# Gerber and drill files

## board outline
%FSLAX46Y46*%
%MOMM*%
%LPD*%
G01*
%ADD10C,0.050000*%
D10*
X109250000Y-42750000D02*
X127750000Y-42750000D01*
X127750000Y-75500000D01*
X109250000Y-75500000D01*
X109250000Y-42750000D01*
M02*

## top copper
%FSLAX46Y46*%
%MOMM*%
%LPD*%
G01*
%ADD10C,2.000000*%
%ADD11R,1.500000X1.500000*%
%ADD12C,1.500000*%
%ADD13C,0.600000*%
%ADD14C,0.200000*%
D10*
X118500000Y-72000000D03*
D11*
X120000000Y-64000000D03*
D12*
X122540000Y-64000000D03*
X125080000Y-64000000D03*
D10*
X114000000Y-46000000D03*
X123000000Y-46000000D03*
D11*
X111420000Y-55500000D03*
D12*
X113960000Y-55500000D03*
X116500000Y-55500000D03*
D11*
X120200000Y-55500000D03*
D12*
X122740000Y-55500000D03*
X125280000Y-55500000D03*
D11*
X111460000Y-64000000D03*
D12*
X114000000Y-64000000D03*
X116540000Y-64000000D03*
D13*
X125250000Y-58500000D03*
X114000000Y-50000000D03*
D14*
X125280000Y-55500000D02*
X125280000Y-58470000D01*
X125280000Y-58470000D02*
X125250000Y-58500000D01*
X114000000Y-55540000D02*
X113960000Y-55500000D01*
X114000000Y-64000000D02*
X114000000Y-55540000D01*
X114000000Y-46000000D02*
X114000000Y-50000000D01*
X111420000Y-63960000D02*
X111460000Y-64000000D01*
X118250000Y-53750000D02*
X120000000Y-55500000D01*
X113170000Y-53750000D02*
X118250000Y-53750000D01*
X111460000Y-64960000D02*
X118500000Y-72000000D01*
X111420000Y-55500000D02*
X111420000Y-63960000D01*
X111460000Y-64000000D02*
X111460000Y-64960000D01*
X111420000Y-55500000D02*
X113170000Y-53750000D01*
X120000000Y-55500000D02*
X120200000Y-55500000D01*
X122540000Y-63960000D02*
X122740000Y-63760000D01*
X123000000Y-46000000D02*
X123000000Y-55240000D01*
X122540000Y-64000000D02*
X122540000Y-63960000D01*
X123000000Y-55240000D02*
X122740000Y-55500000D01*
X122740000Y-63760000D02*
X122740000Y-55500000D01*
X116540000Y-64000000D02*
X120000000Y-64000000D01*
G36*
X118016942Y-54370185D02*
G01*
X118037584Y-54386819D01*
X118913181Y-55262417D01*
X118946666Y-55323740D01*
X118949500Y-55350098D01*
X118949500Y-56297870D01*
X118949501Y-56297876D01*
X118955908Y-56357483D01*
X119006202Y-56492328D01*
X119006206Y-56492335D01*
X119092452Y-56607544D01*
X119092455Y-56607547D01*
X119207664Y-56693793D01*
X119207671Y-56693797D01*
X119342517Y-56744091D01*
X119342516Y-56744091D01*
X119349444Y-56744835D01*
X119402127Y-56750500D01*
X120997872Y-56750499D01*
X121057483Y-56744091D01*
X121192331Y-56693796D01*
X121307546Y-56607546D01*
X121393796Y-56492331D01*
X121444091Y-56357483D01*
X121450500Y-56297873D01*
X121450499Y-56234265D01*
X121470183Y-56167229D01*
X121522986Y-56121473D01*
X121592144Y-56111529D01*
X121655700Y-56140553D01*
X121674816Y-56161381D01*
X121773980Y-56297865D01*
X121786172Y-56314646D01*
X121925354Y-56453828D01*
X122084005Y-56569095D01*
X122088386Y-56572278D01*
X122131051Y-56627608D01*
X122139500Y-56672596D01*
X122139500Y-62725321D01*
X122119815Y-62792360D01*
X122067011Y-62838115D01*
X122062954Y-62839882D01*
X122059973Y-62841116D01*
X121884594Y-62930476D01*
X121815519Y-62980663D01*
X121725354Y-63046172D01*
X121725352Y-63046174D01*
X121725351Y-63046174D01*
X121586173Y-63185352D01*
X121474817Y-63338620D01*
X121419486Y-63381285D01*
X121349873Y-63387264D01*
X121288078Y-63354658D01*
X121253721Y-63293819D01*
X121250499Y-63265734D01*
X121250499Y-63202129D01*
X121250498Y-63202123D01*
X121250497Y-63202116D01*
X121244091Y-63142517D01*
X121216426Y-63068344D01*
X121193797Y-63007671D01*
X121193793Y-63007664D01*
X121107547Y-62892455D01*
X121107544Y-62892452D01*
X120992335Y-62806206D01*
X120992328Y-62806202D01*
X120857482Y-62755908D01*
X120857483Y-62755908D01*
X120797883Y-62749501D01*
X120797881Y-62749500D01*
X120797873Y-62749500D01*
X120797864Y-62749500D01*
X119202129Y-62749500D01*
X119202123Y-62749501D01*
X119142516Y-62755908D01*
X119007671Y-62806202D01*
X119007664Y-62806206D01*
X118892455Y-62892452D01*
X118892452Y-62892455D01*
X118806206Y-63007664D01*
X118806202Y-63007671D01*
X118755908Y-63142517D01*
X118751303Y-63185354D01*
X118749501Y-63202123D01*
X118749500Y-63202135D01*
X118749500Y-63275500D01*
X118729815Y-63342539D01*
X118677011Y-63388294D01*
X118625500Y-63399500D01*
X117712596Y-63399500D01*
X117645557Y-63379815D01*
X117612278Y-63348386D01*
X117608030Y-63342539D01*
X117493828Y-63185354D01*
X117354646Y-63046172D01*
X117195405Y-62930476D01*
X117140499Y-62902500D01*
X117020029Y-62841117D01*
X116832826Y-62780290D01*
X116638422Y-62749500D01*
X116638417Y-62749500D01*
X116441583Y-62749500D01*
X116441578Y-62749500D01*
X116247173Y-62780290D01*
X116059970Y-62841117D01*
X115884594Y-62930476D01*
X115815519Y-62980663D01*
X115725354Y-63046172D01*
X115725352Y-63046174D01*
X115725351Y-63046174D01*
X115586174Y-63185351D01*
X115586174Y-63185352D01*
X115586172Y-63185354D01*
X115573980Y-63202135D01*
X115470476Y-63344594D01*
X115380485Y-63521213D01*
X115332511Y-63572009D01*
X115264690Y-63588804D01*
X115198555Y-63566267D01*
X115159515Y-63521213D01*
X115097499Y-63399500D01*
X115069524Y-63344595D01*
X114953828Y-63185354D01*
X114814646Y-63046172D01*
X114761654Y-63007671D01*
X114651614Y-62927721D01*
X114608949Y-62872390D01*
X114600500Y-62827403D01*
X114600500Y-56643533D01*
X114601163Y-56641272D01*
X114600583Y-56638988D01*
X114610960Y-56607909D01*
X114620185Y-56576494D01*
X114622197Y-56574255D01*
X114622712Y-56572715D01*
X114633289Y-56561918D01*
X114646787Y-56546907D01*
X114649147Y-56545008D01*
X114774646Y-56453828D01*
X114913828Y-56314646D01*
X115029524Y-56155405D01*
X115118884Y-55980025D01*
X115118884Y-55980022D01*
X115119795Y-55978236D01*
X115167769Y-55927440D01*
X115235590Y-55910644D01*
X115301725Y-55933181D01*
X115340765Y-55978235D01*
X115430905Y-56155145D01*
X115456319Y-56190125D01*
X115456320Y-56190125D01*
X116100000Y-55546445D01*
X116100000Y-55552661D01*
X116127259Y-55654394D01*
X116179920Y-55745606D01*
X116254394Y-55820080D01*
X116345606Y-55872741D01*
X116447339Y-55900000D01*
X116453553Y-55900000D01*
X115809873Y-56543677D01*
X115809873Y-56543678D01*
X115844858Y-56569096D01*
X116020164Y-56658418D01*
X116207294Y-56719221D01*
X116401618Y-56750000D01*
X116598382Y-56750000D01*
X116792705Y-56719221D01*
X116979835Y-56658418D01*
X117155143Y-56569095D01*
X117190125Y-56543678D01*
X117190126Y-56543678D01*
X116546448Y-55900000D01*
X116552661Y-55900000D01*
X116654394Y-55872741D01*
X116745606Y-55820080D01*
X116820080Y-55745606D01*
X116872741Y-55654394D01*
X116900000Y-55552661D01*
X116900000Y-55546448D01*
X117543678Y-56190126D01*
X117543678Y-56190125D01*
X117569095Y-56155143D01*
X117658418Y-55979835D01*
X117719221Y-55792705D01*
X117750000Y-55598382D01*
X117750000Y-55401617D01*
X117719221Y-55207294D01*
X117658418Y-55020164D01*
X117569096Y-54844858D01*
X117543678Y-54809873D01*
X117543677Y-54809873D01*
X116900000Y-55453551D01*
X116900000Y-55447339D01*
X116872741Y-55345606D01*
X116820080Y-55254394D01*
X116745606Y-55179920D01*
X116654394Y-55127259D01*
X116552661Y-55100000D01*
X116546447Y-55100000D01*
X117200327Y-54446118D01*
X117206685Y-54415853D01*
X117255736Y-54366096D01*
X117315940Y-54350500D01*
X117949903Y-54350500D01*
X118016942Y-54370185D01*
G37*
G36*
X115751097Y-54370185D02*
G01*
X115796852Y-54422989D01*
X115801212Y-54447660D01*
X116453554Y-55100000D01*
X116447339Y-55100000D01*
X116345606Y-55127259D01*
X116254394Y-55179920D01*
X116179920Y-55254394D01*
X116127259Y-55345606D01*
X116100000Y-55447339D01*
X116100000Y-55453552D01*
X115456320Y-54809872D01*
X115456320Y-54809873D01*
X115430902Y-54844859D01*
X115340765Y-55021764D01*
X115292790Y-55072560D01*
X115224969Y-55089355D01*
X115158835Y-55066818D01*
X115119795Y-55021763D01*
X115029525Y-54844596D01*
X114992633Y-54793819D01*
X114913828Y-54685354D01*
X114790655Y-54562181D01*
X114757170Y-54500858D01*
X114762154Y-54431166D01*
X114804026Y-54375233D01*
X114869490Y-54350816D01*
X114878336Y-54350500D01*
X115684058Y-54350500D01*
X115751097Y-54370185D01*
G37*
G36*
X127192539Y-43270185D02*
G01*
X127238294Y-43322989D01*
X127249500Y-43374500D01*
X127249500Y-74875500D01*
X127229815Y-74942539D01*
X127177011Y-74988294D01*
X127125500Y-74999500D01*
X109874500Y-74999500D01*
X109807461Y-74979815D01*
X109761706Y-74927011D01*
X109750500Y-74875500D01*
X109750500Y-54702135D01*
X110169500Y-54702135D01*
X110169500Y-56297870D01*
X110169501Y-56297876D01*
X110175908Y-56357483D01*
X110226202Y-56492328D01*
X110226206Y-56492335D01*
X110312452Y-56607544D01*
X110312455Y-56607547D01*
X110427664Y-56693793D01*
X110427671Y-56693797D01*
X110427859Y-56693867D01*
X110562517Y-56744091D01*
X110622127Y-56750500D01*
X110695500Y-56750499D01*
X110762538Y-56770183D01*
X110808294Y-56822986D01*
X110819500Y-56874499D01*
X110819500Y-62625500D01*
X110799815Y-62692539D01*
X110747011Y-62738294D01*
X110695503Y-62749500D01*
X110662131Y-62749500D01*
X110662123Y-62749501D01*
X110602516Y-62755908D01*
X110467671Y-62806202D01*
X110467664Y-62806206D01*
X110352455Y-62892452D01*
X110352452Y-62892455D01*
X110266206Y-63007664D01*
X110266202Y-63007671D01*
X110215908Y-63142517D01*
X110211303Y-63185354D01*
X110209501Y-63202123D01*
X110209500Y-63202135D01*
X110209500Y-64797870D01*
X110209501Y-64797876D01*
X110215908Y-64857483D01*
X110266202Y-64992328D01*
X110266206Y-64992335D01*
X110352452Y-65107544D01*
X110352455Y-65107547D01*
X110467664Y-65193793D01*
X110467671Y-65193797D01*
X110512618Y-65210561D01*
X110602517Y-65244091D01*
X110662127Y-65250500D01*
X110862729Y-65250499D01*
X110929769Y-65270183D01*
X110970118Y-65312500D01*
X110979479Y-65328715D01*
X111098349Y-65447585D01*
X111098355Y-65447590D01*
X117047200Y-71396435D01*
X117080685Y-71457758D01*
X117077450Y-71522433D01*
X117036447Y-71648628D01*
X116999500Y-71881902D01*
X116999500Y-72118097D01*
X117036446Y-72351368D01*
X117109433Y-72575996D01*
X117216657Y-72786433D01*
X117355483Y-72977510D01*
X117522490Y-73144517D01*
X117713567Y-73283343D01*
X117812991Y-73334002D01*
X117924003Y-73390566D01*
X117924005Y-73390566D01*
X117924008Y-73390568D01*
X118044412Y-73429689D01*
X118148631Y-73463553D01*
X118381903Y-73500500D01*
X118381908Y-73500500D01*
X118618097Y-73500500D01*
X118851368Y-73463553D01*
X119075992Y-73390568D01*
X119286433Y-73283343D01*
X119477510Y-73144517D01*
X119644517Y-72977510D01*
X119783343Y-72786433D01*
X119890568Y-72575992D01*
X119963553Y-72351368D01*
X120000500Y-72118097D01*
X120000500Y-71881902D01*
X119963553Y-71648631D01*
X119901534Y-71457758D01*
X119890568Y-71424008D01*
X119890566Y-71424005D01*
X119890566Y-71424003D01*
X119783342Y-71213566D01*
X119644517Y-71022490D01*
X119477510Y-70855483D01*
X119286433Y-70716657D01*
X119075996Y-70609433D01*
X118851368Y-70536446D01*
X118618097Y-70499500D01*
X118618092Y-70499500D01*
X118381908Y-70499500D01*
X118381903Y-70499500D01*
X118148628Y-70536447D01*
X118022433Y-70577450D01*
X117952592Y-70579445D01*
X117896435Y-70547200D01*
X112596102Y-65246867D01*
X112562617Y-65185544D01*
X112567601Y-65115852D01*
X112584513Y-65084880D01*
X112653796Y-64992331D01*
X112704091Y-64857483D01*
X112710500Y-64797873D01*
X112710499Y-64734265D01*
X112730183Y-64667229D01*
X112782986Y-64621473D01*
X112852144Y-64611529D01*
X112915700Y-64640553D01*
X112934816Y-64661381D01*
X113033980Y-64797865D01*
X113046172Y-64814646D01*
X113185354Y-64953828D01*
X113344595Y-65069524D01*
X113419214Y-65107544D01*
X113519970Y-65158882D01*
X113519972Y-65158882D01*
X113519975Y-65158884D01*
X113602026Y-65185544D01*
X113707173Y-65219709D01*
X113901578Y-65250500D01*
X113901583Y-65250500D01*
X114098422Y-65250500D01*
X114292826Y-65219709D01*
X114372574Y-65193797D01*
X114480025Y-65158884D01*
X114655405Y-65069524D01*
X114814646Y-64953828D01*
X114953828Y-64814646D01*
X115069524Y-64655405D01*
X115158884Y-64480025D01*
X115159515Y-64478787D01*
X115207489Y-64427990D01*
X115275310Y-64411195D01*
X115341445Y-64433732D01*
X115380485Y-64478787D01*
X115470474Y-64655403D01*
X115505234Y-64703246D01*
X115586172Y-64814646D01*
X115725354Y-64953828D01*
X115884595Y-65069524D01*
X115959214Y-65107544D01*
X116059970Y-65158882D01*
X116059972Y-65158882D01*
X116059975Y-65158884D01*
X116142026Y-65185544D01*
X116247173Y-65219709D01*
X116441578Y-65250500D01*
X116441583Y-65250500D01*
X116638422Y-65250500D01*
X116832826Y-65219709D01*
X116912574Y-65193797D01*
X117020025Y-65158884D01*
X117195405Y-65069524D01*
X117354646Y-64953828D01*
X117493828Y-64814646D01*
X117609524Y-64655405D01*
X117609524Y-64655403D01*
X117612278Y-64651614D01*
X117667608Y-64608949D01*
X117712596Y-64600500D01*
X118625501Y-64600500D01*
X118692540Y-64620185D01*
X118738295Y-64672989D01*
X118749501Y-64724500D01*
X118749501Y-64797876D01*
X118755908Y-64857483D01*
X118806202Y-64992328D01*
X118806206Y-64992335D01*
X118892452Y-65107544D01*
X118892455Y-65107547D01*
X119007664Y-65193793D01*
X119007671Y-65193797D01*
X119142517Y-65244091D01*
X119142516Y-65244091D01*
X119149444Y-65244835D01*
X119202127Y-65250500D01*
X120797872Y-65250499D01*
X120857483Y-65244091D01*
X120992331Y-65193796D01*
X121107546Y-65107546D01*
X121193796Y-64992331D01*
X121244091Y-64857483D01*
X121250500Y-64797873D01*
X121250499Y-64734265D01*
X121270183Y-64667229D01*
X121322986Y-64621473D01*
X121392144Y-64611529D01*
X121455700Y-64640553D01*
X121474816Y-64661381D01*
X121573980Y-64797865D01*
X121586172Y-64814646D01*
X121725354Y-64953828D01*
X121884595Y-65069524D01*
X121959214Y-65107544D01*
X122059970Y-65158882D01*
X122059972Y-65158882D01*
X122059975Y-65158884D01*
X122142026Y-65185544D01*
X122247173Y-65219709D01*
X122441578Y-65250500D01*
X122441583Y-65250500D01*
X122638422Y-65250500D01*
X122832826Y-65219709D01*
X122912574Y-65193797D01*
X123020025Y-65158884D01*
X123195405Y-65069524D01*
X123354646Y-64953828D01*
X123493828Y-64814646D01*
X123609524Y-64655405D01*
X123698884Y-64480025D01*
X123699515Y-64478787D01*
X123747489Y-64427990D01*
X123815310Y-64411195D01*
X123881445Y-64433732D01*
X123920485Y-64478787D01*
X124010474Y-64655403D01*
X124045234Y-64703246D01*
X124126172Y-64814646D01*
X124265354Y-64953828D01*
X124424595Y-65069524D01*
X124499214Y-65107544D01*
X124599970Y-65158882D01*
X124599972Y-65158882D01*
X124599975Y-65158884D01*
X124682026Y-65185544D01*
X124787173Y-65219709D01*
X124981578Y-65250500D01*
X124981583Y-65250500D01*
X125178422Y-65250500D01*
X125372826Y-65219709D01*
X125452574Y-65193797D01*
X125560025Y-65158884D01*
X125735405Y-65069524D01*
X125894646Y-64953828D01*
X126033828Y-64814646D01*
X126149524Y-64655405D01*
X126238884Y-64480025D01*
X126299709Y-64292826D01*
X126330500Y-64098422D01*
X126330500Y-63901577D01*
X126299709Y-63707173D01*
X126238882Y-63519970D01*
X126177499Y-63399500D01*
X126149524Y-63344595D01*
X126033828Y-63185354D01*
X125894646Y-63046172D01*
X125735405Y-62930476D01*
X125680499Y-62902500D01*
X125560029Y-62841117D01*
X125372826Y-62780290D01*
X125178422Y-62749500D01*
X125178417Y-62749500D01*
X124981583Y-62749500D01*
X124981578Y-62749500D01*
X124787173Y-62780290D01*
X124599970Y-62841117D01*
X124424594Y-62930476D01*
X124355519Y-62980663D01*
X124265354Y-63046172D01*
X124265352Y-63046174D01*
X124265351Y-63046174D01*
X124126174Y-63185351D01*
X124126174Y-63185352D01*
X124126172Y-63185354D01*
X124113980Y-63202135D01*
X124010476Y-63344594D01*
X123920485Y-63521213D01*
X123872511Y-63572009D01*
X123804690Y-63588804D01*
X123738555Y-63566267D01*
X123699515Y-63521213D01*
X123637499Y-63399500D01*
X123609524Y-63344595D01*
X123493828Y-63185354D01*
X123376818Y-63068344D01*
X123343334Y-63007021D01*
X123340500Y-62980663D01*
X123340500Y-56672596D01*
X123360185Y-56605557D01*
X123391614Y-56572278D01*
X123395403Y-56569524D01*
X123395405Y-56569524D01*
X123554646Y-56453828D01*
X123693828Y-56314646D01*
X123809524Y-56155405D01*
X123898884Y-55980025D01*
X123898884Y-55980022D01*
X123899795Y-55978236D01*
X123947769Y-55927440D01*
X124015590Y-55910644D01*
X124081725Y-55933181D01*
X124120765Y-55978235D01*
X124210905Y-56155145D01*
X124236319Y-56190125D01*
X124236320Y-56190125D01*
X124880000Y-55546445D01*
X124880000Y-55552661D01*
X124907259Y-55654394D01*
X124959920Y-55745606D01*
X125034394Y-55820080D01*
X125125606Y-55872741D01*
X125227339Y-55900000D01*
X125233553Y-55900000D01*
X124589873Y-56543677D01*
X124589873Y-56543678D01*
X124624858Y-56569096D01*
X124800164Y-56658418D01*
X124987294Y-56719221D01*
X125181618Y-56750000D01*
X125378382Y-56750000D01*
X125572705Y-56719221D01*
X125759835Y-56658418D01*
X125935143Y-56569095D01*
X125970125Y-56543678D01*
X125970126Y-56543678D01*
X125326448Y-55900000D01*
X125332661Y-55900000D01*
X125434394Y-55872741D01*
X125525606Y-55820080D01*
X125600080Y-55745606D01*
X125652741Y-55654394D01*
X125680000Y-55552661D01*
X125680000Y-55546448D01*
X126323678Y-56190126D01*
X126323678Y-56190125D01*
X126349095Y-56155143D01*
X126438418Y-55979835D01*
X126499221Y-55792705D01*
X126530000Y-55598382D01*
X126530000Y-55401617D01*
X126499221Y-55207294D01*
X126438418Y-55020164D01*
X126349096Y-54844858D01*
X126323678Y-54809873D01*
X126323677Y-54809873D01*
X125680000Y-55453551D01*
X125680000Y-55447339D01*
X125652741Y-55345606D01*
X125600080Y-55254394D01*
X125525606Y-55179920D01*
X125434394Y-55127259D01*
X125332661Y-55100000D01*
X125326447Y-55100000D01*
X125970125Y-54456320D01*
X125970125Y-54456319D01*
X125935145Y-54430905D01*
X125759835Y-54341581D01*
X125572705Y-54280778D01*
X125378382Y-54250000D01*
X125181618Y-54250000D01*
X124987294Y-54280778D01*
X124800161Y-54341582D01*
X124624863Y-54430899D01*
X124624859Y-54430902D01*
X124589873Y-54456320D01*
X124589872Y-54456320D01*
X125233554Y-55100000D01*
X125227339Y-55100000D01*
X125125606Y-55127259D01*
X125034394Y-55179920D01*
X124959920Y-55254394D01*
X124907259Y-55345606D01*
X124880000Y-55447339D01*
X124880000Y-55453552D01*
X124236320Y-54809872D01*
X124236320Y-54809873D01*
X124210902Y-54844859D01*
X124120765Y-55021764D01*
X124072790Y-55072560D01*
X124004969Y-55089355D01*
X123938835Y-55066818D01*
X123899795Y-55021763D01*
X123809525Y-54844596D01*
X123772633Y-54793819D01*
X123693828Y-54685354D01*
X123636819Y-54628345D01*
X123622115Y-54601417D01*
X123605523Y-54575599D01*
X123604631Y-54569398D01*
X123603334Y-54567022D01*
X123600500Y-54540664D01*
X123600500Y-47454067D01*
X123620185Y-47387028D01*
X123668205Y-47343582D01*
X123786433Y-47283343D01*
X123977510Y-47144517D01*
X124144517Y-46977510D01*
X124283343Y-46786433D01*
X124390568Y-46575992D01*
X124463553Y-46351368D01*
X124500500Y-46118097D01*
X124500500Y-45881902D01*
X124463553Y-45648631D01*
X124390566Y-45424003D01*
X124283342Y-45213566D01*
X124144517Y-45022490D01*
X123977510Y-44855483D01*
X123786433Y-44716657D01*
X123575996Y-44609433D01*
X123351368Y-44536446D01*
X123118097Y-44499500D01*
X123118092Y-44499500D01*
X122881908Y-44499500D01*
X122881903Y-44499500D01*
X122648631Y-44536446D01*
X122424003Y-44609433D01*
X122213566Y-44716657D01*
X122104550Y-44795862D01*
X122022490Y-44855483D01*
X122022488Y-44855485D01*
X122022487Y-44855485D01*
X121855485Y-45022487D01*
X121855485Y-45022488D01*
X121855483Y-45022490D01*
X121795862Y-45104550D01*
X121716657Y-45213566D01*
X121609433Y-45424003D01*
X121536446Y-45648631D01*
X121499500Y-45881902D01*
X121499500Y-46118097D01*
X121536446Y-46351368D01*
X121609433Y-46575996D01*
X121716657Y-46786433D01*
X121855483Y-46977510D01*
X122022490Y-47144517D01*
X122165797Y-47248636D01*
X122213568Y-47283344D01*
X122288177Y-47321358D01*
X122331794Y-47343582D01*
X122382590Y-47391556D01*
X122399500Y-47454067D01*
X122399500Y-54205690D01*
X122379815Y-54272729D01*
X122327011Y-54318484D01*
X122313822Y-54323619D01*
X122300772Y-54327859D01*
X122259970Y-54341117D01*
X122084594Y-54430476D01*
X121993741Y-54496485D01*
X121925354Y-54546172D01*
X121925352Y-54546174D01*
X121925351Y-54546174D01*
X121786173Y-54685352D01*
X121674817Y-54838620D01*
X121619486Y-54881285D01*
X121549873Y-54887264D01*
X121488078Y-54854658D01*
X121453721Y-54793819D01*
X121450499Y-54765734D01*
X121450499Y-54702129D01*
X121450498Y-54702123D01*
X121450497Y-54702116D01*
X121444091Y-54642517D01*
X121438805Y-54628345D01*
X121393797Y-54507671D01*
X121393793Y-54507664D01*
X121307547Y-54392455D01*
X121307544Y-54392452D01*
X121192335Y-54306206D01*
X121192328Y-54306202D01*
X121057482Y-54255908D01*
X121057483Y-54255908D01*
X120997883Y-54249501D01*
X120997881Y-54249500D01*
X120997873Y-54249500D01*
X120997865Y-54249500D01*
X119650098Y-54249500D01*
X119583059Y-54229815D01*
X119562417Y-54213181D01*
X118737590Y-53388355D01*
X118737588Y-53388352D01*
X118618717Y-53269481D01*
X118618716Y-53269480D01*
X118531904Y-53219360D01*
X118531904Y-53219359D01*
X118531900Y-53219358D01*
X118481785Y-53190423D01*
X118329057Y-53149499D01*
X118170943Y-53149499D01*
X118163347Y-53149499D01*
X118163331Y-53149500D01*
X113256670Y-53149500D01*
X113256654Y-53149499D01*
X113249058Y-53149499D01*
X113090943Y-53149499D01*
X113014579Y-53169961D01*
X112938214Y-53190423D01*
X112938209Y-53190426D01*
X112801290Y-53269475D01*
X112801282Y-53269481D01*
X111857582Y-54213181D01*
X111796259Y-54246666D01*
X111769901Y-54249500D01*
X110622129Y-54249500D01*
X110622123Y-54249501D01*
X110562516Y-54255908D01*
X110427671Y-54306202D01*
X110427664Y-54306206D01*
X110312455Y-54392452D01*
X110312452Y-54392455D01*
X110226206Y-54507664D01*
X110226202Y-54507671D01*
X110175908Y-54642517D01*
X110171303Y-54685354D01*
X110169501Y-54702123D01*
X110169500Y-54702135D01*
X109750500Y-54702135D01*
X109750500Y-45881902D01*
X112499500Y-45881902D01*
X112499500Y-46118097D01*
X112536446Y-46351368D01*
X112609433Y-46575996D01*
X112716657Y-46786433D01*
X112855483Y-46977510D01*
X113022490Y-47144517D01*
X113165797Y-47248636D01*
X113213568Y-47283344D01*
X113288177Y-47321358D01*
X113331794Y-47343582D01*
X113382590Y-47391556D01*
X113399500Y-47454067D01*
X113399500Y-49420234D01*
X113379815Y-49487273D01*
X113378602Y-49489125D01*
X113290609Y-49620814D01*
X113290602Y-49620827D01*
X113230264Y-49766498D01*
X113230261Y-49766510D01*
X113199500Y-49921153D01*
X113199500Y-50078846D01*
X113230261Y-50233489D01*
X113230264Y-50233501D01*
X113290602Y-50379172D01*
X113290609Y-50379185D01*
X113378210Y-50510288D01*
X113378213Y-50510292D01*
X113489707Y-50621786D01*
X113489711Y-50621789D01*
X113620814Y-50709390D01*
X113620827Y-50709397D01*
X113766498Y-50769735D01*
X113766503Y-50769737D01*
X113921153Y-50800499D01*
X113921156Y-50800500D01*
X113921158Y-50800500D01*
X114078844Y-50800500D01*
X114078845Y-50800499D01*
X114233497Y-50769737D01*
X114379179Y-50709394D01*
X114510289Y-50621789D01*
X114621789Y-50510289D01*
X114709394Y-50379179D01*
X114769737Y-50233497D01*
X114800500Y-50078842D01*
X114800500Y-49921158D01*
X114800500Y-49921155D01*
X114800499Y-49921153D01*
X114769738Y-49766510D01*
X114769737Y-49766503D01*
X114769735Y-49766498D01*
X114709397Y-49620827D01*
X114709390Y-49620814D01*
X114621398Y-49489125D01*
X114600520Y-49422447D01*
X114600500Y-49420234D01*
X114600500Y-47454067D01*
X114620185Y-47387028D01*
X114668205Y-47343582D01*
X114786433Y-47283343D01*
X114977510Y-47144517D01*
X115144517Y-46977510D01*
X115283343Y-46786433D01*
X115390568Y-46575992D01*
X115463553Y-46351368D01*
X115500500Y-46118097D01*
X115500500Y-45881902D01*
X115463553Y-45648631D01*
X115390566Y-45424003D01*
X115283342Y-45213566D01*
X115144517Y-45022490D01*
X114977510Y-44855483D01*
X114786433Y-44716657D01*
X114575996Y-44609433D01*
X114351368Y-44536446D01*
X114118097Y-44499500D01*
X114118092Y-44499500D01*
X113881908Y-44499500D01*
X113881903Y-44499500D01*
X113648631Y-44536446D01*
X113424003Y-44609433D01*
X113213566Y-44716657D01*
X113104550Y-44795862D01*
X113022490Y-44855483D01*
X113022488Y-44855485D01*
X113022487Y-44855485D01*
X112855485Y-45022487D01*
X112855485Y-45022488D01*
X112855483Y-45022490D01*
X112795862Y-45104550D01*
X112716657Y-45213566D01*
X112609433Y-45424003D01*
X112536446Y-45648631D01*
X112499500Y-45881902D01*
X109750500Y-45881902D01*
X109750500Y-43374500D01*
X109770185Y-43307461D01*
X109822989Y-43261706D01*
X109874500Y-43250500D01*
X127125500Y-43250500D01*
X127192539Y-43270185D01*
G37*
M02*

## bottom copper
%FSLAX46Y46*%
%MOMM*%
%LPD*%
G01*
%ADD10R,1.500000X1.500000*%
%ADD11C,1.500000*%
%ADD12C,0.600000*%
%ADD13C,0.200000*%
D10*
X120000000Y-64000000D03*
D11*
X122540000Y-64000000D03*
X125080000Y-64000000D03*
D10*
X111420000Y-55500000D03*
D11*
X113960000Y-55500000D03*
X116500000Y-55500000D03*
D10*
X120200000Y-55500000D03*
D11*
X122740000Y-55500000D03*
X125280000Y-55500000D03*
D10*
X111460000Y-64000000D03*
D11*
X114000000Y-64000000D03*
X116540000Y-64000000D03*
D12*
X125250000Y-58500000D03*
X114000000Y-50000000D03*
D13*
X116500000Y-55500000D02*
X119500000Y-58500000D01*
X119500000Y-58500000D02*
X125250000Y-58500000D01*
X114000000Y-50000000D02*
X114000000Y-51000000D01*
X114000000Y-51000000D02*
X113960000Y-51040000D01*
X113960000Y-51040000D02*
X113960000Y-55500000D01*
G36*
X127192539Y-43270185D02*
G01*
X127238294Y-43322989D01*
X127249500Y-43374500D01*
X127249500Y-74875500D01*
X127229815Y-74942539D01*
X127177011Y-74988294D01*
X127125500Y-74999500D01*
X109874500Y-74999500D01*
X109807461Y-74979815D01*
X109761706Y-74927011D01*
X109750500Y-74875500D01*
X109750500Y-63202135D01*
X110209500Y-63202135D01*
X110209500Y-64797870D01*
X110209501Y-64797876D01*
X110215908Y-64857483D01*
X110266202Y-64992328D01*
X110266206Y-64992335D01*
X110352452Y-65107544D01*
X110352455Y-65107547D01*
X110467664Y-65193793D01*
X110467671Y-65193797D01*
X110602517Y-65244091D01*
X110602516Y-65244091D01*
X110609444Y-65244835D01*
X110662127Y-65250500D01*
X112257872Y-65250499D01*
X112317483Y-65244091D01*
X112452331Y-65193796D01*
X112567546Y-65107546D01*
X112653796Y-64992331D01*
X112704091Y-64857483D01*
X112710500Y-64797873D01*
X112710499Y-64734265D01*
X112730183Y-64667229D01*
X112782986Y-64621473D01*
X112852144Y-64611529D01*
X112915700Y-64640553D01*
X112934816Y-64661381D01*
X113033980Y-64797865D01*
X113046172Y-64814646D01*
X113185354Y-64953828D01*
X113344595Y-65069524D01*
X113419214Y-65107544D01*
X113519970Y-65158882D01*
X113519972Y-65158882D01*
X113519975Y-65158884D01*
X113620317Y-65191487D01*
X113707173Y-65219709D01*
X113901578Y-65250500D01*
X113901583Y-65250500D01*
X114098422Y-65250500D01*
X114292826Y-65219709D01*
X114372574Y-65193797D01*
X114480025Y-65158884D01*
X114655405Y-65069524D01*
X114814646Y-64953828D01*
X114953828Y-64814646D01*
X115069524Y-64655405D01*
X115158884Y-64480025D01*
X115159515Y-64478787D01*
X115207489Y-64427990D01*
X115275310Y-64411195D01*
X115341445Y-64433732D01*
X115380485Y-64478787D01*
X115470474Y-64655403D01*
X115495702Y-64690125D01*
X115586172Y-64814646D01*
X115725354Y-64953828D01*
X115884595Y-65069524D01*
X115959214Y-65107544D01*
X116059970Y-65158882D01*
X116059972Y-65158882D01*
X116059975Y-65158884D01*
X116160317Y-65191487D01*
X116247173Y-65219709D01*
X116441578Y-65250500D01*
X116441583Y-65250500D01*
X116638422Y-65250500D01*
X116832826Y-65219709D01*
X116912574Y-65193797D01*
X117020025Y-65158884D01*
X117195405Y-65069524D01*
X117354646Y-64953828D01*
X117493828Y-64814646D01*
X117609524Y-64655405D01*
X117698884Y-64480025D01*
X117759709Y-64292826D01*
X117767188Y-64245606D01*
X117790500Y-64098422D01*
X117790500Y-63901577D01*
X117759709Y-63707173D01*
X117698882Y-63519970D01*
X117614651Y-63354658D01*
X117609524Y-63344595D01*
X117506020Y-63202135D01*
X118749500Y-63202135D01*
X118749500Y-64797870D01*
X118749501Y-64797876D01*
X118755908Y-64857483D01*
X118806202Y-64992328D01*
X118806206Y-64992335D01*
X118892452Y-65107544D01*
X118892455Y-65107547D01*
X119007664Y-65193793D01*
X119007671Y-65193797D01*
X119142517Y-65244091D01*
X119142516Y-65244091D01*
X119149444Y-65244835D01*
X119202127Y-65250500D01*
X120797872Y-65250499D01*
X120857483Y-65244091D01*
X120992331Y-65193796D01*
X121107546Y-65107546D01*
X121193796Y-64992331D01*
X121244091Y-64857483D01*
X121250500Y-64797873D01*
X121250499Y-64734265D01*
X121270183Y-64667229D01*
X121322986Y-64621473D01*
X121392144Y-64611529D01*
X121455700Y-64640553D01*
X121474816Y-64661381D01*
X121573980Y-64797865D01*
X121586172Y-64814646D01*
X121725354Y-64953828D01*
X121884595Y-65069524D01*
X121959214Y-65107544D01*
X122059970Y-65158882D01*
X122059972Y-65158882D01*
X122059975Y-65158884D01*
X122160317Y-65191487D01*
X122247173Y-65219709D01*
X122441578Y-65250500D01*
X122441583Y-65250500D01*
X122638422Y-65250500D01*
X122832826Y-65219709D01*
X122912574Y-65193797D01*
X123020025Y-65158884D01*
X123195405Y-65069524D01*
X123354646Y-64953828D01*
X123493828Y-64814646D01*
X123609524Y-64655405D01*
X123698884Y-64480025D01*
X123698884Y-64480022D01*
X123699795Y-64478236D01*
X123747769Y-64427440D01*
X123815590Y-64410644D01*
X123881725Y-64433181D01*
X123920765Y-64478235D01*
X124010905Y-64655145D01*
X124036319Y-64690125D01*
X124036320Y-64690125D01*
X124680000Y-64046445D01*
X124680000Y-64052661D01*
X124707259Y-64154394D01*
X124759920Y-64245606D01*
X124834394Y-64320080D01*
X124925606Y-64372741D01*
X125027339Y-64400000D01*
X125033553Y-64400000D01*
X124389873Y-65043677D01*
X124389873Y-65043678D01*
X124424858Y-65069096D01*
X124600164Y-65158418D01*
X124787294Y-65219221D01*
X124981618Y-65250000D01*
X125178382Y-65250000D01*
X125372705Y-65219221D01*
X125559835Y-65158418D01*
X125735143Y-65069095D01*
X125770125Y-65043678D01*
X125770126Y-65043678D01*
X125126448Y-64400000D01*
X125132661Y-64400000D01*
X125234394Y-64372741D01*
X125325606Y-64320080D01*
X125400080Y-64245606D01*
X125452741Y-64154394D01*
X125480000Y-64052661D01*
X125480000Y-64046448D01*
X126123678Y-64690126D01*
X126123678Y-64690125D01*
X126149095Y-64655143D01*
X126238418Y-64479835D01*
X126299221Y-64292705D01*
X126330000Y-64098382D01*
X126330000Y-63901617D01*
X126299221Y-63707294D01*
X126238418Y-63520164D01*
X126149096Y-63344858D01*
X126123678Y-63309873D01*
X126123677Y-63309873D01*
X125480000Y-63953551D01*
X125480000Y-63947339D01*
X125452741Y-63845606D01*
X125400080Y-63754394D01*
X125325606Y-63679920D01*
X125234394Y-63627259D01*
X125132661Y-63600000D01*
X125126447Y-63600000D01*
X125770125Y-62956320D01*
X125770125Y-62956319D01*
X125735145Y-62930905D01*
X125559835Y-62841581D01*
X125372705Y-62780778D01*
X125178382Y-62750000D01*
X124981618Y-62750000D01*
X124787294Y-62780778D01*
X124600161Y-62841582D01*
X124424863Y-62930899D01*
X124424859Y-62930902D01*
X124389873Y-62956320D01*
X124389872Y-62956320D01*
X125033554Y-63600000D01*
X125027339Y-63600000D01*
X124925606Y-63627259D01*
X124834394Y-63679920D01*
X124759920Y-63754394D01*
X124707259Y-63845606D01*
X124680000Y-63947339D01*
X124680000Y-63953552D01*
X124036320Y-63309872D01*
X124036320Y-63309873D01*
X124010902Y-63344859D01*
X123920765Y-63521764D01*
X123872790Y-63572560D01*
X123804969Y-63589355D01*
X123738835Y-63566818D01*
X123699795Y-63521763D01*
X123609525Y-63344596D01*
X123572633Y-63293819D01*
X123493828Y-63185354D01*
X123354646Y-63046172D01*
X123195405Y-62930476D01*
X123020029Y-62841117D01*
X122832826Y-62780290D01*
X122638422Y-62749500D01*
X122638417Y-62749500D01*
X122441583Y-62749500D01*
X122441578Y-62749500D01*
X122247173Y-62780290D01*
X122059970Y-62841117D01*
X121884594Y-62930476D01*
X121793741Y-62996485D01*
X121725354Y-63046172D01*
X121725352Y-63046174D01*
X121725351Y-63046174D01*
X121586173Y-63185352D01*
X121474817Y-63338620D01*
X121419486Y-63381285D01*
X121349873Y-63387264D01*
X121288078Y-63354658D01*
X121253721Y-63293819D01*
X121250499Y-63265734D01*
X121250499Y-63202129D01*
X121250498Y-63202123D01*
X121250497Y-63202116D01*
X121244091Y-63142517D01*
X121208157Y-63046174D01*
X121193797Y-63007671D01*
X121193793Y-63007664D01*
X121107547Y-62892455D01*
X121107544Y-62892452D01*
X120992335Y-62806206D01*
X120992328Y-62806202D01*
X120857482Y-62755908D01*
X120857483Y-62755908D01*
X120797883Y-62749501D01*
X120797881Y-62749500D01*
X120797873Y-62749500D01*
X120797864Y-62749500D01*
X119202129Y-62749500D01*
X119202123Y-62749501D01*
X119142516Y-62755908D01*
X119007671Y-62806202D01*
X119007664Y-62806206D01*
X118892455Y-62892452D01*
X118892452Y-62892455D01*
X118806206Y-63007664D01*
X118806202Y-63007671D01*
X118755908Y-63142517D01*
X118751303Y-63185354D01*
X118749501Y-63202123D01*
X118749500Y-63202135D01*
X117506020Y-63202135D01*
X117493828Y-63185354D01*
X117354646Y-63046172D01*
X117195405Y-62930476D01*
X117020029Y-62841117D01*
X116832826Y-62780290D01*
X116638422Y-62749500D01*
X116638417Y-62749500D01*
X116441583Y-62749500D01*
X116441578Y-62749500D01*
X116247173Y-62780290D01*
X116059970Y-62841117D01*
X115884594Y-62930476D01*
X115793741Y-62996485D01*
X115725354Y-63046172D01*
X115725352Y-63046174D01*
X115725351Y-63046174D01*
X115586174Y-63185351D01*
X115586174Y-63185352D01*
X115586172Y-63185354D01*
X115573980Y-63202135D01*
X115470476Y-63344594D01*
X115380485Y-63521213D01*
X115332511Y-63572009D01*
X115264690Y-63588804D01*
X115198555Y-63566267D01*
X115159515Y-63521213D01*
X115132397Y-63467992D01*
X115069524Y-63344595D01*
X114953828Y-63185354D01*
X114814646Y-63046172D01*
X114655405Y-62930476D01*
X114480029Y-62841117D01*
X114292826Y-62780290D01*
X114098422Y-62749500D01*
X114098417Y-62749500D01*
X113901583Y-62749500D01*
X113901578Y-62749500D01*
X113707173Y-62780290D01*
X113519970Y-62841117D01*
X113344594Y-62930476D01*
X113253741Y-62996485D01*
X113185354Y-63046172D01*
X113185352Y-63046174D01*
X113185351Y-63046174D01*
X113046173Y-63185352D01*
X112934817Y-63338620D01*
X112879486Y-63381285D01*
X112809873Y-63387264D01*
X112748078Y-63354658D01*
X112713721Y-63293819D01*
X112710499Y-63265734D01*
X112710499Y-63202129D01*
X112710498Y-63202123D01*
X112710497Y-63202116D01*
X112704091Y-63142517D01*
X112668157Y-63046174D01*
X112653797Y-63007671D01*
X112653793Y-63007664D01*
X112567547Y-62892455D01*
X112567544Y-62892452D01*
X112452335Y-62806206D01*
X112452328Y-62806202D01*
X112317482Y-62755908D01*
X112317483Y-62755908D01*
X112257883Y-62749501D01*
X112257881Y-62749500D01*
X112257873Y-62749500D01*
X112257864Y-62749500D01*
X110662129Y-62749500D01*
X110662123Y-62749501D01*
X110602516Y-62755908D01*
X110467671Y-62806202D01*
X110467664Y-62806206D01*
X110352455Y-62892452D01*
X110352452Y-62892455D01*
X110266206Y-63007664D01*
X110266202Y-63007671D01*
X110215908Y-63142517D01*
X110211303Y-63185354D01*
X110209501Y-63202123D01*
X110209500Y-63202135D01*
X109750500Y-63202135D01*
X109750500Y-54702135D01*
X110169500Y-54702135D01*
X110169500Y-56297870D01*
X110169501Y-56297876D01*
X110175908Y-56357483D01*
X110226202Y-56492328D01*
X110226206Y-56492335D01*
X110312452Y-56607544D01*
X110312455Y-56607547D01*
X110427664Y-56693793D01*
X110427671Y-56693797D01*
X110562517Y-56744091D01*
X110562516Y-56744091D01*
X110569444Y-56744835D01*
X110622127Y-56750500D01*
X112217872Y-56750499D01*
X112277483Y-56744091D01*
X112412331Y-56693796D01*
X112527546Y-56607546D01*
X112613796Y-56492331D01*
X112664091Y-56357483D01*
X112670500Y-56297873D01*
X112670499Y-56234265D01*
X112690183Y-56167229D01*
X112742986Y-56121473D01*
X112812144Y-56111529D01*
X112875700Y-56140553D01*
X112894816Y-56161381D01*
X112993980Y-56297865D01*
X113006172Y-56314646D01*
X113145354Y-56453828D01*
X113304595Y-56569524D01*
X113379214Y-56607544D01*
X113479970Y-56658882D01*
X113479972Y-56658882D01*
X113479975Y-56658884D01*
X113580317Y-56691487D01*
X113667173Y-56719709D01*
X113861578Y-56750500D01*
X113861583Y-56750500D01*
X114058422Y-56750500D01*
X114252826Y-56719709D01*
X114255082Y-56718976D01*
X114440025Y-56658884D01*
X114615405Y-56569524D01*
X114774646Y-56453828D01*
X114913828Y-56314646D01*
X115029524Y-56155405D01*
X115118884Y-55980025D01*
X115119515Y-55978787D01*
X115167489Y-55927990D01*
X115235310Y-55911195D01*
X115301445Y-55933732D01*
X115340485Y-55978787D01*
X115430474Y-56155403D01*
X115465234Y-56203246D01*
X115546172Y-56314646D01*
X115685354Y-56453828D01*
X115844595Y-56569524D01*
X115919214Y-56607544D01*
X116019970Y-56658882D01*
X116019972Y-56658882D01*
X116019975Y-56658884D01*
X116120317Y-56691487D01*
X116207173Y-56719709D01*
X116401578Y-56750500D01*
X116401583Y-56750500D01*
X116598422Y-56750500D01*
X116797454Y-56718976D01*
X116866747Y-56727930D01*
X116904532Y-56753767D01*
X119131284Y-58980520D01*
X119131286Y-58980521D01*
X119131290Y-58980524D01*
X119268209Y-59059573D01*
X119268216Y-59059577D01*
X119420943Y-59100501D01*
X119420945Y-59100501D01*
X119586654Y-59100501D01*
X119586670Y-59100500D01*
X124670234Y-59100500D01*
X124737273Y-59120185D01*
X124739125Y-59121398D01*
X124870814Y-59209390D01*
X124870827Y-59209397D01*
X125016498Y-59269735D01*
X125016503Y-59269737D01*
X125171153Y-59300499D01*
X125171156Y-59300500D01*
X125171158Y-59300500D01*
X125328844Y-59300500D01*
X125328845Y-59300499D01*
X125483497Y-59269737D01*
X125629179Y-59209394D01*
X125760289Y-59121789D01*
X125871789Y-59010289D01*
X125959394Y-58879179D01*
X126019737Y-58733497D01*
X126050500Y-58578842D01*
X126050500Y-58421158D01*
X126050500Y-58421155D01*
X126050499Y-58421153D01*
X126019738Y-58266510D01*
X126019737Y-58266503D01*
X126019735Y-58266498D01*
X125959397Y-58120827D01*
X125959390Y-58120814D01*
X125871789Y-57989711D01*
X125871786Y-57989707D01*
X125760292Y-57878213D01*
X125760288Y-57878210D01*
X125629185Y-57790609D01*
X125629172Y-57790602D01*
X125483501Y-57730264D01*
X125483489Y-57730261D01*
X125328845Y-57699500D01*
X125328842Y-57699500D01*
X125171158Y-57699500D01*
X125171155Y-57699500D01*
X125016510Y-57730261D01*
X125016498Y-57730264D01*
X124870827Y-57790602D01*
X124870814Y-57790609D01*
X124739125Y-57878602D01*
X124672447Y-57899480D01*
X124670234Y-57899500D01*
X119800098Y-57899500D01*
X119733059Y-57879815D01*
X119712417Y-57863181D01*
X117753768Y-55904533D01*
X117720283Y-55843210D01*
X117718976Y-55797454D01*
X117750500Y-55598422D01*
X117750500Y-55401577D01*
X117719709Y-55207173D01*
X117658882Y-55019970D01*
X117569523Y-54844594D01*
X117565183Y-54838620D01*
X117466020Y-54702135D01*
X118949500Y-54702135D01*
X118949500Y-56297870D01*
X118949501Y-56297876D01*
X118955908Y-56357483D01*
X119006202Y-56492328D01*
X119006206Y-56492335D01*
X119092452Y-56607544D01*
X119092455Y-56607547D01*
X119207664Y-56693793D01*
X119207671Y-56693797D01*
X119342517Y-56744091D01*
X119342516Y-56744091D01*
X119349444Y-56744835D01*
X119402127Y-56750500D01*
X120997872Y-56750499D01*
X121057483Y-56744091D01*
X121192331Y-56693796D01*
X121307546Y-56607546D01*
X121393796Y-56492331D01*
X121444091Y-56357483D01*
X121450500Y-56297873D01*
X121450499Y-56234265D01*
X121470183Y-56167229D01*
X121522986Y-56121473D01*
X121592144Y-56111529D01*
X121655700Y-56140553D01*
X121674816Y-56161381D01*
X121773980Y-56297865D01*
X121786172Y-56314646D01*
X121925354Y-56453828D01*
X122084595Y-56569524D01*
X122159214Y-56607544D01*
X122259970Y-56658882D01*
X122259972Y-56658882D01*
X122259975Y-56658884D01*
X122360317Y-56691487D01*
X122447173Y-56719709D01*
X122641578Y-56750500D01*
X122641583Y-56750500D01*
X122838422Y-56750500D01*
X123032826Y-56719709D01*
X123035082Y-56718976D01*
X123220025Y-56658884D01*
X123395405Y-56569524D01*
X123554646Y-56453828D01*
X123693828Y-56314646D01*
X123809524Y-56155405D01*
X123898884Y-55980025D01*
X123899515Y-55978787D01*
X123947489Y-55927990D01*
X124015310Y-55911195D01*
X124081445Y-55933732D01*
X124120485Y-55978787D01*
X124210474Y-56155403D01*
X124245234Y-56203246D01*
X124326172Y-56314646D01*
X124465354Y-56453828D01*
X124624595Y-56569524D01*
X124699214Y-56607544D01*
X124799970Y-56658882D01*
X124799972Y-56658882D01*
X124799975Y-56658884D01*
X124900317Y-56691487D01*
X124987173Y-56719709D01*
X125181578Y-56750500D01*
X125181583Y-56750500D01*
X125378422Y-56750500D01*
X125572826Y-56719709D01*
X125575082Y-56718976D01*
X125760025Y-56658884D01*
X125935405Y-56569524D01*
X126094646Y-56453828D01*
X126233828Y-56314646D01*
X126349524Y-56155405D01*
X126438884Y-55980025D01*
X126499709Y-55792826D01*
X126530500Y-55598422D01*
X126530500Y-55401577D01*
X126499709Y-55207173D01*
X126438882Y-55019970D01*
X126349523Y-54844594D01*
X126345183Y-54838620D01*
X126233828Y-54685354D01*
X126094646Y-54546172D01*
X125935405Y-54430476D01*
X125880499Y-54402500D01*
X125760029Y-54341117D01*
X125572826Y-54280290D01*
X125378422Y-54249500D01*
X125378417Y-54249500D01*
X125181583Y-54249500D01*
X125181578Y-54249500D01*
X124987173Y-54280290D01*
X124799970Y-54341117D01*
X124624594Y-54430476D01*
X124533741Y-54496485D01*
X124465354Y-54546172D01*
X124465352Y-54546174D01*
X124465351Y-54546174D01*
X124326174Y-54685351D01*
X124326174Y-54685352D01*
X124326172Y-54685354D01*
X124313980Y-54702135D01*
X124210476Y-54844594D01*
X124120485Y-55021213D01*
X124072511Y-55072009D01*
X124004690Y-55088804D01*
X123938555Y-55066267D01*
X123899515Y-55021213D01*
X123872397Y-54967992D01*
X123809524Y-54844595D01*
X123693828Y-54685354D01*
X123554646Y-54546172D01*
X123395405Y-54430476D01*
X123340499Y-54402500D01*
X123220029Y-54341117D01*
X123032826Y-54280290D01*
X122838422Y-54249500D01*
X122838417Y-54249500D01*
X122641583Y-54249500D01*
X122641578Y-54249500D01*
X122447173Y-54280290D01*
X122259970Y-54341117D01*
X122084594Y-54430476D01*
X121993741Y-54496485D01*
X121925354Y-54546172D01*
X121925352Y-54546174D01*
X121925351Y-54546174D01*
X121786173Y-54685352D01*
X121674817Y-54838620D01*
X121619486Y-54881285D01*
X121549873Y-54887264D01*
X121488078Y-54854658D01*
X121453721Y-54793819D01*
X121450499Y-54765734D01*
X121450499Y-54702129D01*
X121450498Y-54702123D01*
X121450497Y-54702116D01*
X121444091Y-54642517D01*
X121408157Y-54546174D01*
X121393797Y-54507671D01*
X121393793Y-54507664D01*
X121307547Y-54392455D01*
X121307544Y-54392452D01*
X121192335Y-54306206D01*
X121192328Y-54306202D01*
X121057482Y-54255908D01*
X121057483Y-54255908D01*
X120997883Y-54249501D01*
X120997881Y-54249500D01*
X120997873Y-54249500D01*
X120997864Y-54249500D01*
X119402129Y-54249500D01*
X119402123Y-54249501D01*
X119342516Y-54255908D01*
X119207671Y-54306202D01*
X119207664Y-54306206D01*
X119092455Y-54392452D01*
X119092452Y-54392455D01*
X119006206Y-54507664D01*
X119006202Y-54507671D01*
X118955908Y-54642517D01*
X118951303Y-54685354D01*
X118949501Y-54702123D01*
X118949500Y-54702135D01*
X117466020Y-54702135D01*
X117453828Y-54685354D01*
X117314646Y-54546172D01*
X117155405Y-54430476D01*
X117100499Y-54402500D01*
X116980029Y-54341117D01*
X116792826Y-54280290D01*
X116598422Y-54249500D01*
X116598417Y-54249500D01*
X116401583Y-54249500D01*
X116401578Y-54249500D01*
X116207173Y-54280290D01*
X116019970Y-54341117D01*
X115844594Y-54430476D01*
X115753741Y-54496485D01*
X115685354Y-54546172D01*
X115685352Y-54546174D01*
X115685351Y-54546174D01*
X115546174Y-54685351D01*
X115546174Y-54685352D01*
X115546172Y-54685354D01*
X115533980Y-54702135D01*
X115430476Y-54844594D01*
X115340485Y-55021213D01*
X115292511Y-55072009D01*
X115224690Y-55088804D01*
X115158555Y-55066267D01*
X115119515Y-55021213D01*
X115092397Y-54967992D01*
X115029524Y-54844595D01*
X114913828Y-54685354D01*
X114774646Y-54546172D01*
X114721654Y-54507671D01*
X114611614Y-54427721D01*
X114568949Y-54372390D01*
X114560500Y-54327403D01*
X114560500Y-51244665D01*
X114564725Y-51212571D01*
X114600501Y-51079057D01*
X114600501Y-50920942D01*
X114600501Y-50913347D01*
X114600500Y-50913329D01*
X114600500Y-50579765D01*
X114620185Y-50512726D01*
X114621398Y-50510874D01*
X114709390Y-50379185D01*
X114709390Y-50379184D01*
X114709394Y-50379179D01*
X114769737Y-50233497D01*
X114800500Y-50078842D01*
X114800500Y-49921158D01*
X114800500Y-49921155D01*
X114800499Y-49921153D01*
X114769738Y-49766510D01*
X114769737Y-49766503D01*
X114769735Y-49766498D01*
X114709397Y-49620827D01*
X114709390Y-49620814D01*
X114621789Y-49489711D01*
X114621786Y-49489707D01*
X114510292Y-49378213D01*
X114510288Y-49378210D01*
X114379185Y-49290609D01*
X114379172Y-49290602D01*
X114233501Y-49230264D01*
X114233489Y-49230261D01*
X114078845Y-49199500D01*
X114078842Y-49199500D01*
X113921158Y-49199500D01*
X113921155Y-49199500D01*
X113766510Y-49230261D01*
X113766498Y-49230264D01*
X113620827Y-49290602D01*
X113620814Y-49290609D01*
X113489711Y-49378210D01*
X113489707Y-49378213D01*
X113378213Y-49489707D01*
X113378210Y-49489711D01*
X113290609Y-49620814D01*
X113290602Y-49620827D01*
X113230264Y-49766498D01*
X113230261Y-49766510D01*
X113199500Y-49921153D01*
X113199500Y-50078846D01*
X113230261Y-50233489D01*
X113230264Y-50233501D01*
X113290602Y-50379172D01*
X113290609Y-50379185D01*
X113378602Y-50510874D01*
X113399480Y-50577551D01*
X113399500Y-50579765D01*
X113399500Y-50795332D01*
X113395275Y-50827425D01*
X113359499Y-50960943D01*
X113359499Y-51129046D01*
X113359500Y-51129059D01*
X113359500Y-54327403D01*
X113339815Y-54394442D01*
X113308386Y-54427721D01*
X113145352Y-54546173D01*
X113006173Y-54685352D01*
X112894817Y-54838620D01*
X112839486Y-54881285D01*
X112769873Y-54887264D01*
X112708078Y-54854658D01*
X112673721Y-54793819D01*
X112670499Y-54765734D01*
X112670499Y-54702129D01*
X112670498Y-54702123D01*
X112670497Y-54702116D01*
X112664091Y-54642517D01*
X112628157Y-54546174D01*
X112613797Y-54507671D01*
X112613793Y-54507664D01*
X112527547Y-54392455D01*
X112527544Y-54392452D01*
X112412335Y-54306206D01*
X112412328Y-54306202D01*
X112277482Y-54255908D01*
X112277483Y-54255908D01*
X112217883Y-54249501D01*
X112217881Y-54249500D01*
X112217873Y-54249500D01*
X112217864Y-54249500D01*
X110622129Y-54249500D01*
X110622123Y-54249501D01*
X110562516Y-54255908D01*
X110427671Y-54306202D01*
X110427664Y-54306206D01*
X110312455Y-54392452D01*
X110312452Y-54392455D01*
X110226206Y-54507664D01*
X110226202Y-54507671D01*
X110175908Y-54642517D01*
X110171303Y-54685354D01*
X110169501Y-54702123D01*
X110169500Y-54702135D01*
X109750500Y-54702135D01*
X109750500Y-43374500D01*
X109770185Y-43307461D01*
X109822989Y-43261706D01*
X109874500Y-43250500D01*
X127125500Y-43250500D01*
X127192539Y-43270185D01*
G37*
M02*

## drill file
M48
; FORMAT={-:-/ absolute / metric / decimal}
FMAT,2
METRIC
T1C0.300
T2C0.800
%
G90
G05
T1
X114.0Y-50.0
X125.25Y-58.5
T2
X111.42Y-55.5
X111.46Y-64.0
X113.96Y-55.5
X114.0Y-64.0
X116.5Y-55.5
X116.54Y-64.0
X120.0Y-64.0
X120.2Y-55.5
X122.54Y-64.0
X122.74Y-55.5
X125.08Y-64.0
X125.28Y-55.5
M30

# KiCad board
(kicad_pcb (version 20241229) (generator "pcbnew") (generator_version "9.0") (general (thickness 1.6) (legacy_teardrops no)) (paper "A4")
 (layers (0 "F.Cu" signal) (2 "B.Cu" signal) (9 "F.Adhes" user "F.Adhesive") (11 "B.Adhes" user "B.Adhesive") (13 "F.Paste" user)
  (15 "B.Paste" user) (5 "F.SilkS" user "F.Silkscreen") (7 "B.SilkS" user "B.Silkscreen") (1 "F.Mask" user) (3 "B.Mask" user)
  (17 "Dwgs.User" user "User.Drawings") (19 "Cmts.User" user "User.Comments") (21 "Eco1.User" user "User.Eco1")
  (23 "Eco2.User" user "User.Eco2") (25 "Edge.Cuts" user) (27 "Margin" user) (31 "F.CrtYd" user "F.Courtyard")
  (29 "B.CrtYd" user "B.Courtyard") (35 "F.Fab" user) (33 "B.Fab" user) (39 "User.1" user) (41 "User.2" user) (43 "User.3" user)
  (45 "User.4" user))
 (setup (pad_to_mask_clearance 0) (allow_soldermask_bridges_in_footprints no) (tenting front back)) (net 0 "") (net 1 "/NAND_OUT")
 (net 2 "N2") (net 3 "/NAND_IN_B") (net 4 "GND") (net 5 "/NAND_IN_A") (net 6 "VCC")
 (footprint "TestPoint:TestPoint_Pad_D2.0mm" (layer "F.Cu") (at 118.5 72)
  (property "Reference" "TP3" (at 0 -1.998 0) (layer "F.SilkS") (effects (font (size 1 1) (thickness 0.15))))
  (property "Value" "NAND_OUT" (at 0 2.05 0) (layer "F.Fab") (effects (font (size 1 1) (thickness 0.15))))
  (pad "1" smd circle (at 0 0) (size 2 2) (layers "F.Cu" "F.Mask") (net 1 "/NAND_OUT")))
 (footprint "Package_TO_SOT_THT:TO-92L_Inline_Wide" (layer "F.Cu") (at 120 64)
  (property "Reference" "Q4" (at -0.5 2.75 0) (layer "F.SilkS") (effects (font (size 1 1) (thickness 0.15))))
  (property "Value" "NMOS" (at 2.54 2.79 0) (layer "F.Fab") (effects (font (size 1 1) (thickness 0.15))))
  (pad "1" thru_hole rect (at 0 0) (size 1.5 1.5) (drill 0.8) (layers "*.Cu" "*.Mask") (remove_unused_layers no) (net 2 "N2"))
  (pad "2" thru_hole circle (at 2.54 0) (size 1.5 1.5) (drill 0.8) (layers "*.Cu" "*.Mask") (remove_unused_layers no) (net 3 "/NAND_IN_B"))
  (pad "3" thru_hole circle (at 5.08 0) (size 1.5 1.5) (drill 0.8) (layers "*.Cu" "*.Mask") (remove_unused_layers no) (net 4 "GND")))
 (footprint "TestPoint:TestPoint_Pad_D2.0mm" (layer "F.Cu") (at 114 46)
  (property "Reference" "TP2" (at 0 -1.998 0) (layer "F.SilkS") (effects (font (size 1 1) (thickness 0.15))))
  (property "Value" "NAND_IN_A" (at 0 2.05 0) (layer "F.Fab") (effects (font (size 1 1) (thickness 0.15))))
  (pad "1" smd circle (at 0 0) (size 2 2) (layers "F.Cu" "F.Mask") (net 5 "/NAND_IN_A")))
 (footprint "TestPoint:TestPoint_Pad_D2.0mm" (layer "F.Cu") (at 123 46)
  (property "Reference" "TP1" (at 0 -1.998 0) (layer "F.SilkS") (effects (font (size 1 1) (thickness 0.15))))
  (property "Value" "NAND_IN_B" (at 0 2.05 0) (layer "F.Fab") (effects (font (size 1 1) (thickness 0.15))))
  (pad "1" smd circle (at 0 0) (size 2 2) (layers "F.Cu" "F.Mask") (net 3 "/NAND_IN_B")))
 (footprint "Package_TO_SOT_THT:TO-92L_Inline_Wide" (layer "F.Cu") (at 111.42 55.5)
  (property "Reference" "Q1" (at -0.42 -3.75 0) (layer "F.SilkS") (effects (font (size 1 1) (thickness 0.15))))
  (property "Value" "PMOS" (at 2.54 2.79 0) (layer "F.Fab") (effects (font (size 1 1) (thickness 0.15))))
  (pad "1" thru_hole rect (at 0 0) (size 1.5 1.5) (drill 0.8) (layers "*.Cu" "*.Mask") (remove_unused_layers no) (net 1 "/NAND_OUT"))
  (pad "2" thru_hole circle (at 2.54 0) (size 1.5 1.5) (drill 0.8) (layers "*.Cu" "*.Mask") (remove_unused_layers no) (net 5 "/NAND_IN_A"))
  (pad "3" thru_hole circle (at 5.08 0) (size 1.5 1.5) (drill 0.8) (layers "*.Cu" "*.Mask") (remove_unused_layers no) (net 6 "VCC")))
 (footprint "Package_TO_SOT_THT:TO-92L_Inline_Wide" (layer "F.Cu") (at 120.2 55.5)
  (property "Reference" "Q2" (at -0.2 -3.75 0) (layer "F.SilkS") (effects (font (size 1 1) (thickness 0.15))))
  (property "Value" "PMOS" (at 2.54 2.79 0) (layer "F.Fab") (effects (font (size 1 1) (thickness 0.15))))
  (pad "1" thru_hole rect (at 0 0) (size 1.5 1.5) (drill 0.8) (layers "*.Cu" "*.Mask") (remove_unused_layers no) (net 1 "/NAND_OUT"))
  (pad "2" thru_hole circle (at 2.54 0) (size 1.5 1.5) (drill 0.8) (layers "*.Cu" "*.Mask") (remove_unused_layers no) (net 3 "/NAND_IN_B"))
  (pad "3" thru_hole circle (at 5.08 0) (size 1.5 1.5) (drill 0.8) (layers "*.Cu" "*.Mask") (remove_unused_layers no) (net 6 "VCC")))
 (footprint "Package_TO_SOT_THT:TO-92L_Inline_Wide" (layer "F.Cu") (at 111.46 64)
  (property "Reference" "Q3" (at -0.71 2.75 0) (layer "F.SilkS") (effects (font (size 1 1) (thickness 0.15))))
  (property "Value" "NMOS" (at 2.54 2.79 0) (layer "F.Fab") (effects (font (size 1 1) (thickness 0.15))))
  (pad "1" thru_hole rect (at 0 0) (size 1.5 1.5) (drill 0.8) (layers "*.Cu" "*.Mask") (remove_unused_layers no) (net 1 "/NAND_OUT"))
  (pad "2" thru_hole circle (at 2.54 0) (size 1.5 1.5) (drill 0.8) (layers "*.Cu" "*.Mask") (remove_unused_layers no) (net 5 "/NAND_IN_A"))
  (pad "3" thru_hole circle (at 5.08 0) (size 1.5 1.5) (drill 0.8) (layers "*.Cu" "*.Mask") (remove_unused_layers no) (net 2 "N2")))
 (gr_rect (start 109.25 42.75) (end 127.75 75.5) (stroke (width 0.05) (type default)) (fill no) (layer "Edge.Cuts"))
 (segment (start 125.28 55.5) (end 125.28 58.47) (width 0.2) (layer "F.Cu") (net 6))
 (segment (start 125.28 58.47) (end 125.25 58.5) (width 0.2) (layer "F.Cu") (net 6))
 (via (at 125.25 58.5) (size 0.6) (drill 0.3) (layers "F.Cu" "B.Cu") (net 6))
 (segment (start 116.5 55.5) (end 119.5 58.5) (width 0.2) (layer "B.Cu") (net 6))
 (segment (start 119.5 58.5) (end 125.25 58.5) (width 0.2) (layer "B.Cu") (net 6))
 (segment (start 114 55.54) (end 113.96 55.5) (width 0.2) (layer "F.Cu") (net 5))
 (segment (start 114 64) (end 114 55.54) (width 0.2) (layer "F.Cu") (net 5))
 (segment (start 114 46) (end 114 50) (width 0.2) (layer "F.Cu") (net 5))
 (via (at 114 50) (size 0.6) (drill 0.3) (layers "F.Cu" "B.Cu") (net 5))
 (segment (start 114 50) (end 114 51) (width 0.2) (layer "B.Cu") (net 5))
 (segment (start 114 51) (end 113.96 51.04) (width 0.2) (layer "B.Cu") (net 5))
 (segment (start 113.96 51.04) (end 113.96 55.5) (width 0.2) (layer "B.Cu") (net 5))
 (segment (start 111.42 63.96) (end 111.46 64) (width 0.2) (layer "F.Cu") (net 1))
 (segment (start 118.25 53.75) (end 120 55.5) (width 0.2) (layer "F.Cu") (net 1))
 (segment (start 113.17 53.75) (end 118.25 53.75) (width 0.2) (layer "F.Cu") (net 1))
 (segment (start 111.46 64.96) (end 118.5 72) (width 0.2) (layer "F.Cu") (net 1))
 (segment (start 111.42 55.5) (end 111.42 63.96) (width 0.2) (layer "F.Cu") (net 1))
 (segment (start 111.46 64) (end 111.46 64.96) (width 0.2) (layer "F.Cu") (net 1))
 (segment (start 111.42 55.5) (end 113.17 53.75) (width 0.2) (layer "F.Cu") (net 1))
 (segment (start 120 55.5) (end 120.2 55.5) (width 0.2) (layer "F.Cu") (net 1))
 (segment (start 122.54 63.96) (end 122.74 63.76) (width 0.2) (layer "F.Cu") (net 3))
 (segment (start 123 46) (end 123 55.24) (width 0.2) (layer "F.Cu") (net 3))
 (segment (start 122.54 64) (end 122.54 63.96) (width 0.2) (layer "F.Cu") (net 3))
 (segment (start 123 55.24) (end 122.74 55.5) (width 0.2) (layer "F.Cu") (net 3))
 (segment (start 122.74 63.76) (end 122.74 55.5) (width 0.2) (layer "F.Cu") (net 3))
 (segment (start 116.54 64) (end 120 64) (width 0.2) (layer "F.Cu") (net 2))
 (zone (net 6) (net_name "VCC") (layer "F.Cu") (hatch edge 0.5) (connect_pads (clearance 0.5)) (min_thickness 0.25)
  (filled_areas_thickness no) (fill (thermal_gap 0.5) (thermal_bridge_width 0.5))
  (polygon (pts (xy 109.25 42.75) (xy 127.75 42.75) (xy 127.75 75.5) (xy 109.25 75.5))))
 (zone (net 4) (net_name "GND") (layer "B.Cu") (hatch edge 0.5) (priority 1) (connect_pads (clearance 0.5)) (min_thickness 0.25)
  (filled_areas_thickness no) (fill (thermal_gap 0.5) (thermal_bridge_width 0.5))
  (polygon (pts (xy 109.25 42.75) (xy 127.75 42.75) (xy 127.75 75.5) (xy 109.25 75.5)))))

